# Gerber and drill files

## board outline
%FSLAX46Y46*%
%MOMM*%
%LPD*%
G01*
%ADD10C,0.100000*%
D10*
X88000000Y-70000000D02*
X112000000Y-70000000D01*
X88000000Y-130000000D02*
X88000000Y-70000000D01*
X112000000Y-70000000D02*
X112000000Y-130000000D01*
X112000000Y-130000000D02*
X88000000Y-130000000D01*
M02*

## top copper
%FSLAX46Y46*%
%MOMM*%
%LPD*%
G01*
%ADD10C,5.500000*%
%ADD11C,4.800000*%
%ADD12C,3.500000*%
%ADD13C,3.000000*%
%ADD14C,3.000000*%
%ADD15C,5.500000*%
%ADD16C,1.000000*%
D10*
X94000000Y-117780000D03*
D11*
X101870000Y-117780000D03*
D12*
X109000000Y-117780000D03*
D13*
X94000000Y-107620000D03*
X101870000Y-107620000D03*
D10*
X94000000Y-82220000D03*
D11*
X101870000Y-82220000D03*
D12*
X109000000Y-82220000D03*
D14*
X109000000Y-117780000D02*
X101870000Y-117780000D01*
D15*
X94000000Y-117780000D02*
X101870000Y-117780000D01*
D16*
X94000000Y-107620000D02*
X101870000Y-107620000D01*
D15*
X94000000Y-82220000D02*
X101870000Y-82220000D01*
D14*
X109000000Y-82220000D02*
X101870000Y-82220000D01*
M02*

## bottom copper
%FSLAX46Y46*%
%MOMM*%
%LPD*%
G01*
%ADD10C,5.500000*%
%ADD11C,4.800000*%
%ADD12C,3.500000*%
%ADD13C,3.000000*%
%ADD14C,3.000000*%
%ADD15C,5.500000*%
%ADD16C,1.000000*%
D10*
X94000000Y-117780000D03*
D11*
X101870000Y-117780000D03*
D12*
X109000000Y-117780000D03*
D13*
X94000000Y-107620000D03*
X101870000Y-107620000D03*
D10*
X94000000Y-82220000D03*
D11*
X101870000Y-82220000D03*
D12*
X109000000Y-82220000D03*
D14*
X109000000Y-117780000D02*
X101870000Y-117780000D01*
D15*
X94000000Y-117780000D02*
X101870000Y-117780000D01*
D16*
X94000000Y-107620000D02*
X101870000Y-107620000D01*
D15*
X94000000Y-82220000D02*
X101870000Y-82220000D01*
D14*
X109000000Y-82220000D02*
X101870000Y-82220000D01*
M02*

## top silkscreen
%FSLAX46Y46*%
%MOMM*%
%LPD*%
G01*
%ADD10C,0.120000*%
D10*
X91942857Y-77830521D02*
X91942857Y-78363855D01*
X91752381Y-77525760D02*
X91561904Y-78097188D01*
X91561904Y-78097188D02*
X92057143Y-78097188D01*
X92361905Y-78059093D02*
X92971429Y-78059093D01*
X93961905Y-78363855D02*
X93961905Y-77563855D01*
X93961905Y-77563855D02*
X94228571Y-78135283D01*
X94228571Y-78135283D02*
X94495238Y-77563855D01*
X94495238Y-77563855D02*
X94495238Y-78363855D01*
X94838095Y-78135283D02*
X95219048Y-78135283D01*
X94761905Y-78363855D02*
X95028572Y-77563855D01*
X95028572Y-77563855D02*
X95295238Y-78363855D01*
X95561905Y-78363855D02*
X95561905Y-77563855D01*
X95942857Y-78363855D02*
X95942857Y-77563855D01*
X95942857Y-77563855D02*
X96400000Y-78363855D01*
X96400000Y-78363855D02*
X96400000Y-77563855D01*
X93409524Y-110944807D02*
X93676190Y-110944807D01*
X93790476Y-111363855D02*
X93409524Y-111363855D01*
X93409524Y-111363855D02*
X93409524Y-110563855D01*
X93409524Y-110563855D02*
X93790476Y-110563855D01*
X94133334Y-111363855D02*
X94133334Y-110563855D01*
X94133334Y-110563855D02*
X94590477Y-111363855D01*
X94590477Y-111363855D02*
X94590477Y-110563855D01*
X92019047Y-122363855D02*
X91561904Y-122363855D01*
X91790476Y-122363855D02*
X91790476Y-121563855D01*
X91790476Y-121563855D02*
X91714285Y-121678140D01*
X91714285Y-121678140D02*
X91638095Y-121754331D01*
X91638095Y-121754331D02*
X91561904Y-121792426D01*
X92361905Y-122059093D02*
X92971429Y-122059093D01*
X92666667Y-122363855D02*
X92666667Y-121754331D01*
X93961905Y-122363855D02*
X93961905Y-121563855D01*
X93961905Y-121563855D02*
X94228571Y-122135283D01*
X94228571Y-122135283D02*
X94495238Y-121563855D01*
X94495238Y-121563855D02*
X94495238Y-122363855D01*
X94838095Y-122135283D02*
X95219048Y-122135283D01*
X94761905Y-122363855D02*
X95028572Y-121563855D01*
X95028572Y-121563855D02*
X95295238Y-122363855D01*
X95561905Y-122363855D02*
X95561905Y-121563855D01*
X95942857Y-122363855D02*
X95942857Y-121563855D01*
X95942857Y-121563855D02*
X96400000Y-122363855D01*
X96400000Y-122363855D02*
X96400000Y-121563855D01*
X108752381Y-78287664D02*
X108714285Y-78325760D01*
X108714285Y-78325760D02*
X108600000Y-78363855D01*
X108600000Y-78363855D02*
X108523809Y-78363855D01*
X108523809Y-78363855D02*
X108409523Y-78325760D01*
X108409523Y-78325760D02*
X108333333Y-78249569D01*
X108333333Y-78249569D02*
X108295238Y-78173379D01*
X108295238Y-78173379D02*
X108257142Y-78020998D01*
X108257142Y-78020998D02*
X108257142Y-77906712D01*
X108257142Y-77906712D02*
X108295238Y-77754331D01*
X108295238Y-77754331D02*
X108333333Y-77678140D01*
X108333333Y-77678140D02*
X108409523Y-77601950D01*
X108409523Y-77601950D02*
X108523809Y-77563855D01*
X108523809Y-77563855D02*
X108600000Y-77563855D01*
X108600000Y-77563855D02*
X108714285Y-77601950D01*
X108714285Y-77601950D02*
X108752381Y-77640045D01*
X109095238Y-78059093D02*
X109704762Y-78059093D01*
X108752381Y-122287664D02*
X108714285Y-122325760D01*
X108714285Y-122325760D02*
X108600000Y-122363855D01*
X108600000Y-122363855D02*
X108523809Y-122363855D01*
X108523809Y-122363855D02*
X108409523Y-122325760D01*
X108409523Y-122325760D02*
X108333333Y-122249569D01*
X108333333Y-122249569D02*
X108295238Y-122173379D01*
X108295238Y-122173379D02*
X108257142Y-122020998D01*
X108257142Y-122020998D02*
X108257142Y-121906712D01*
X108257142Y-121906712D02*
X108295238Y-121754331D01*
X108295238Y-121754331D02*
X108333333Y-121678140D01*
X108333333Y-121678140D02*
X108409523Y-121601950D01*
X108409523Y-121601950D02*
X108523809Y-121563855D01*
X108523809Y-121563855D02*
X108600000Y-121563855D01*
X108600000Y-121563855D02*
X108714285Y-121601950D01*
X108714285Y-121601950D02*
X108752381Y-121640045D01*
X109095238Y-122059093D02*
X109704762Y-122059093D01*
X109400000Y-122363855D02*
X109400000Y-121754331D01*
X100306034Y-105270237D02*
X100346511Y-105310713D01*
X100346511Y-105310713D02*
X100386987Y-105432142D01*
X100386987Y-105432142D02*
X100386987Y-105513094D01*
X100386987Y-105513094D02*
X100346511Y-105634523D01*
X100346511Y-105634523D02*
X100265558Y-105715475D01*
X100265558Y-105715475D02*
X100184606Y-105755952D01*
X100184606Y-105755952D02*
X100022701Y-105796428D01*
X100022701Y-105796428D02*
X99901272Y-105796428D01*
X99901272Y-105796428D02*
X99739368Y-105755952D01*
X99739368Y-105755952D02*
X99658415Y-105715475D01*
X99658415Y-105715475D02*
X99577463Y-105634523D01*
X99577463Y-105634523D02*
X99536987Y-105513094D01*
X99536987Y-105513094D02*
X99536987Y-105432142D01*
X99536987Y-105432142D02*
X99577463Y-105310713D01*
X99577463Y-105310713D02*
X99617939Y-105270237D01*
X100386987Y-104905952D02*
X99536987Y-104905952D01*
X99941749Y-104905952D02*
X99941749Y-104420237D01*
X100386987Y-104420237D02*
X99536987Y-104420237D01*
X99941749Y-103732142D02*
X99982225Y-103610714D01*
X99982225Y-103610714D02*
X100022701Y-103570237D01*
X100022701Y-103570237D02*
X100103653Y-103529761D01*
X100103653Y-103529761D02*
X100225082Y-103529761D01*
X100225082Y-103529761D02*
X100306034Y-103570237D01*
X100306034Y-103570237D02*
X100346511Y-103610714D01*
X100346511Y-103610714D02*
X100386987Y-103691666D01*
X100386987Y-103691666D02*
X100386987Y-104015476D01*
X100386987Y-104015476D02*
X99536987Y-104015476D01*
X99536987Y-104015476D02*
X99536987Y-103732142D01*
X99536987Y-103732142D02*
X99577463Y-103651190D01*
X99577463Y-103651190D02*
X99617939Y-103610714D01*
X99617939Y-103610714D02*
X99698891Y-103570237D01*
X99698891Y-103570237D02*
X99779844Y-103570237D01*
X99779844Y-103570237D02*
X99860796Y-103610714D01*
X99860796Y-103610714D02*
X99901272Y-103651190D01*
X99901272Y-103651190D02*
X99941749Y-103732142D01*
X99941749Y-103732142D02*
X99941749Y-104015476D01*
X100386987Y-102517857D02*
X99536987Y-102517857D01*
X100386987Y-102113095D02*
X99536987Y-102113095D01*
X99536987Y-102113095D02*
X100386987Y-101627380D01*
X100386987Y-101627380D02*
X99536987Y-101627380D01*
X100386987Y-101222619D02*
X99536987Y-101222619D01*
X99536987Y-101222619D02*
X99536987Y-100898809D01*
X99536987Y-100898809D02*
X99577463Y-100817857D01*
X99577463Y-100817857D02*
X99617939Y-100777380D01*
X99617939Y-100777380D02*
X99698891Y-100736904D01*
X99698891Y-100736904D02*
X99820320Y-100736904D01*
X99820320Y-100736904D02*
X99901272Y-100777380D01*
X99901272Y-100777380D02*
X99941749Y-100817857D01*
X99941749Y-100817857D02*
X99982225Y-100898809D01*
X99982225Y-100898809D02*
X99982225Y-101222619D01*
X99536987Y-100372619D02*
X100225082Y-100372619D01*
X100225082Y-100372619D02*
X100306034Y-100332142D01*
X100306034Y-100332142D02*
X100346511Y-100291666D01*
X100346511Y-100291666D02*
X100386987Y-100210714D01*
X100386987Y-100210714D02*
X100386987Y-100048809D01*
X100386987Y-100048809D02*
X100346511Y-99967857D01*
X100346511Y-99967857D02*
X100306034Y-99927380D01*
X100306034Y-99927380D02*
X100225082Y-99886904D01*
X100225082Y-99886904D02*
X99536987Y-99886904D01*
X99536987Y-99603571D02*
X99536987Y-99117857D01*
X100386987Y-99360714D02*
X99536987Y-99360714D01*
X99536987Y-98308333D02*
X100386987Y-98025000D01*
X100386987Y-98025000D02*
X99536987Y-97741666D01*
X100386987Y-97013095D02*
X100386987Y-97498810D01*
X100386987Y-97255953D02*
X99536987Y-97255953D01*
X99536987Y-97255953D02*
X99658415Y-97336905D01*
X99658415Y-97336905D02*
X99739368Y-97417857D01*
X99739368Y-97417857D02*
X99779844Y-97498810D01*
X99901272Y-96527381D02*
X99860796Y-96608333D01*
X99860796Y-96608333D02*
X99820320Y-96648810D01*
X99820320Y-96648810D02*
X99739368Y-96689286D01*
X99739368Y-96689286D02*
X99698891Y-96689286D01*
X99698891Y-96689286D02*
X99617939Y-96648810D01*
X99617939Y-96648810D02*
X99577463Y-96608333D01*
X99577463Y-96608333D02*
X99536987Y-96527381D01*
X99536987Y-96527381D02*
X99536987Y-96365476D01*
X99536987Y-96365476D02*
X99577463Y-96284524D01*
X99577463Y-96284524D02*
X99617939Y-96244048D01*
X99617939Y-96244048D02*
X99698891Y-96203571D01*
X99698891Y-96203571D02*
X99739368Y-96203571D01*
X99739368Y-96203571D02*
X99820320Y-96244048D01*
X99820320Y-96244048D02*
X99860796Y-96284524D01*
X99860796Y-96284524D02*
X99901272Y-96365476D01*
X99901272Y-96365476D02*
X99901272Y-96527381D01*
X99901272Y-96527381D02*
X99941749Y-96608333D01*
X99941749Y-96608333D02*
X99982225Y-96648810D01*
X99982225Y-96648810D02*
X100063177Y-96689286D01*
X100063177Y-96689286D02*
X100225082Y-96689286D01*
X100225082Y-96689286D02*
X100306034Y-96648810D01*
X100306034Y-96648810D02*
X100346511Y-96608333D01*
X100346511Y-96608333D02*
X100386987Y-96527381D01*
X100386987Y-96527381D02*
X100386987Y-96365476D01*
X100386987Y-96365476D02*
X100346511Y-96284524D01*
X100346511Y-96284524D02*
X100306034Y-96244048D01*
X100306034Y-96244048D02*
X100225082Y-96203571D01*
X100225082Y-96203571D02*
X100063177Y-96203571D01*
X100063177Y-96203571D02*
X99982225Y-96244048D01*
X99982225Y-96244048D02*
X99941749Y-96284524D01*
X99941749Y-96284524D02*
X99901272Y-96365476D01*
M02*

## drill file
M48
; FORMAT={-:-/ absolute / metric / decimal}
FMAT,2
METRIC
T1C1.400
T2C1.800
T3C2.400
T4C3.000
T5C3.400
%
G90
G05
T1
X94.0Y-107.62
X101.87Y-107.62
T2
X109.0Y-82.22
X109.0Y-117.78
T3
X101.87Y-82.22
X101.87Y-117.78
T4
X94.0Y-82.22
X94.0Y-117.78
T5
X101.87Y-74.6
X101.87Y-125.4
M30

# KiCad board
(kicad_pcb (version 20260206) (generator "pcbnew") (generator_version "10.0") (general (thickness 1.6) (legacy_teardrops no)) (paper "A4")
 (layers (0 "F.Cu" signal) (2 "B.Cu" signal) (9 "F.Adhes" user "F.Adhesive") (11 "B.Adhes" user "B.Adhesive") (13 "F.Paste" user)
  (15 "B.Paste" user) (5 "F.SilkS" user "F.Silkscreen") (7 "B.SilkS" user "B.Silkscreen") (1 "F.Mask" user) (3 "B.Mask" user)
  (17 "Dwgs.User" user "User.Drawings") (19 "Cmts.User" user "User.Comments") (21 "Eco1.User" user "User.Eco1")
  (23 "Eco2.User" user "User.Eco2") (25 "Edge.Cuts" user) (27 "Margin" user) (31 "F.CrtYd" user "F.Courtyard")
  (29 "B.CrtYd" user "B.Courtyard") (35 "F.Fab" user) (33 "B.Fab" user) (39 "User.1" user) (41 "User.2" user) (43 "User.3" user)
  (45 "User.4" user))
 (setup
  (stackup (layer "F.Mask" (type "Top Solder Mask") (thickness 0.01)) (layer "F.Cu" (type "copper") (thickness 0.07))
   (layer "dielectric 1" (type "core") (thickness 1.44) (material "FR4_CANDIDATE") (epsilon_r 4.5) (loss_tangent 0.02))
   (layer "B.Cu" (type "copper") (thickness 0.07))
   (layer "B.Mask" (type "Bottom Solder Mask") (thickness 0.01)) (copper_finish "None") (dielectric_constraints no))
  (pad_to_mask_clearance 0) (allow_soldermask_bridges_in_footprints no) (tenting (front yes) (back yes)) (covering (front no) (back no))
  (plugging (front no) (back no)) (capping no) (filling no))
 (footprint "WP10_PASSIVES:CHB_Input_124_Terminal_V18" (layer "F.Cu") (at 100 100)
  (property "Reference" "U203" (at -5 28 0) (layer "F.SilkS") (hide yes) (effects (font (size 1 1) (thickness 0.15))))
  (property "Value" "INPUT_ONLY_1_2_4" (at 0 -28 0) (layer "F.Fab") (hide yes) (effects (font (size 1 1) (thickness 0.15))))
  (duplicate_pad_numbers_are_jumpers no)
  (pad "" np_thru_hole circle (at 1.87 -25.4) (size 3.4 3.4) (drill 3.4) (layers "*.Cu" "*.Mask"))
  (pad "" np_thru_hole circle (at 1.87 25.4) (size 3.4 3.4) (drill 3.4) (layers "*.Cu" "*.Mask"))
  (pad "1" thru_hole circle (at -6 17.78) (size 5.5 5.5) (drill 3) (layers "*.Cu" "*.Mask") (remove_unused_layers no)
   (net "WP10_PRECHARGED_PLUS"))
  (pad "1" thru_hole circle (at 1.87 17.78) (size 4.8 4.8) (drill 2.4) (layers "*.Cu" "*.Mask") (remove_unused_layers no)
   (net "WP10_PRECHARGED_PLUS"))
  (pad "1" thru_hole circle (at 9 17.78) (size 3.5 3.5) (drill 1.8) (layers "*.Cu" "*.Mask") (remove_unused_layers no)
   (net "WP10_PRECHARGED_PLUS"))
  (pad "2" thru_hole circle (at -6 7.62) (size 3 3) (drill 1.4) (layers "*.Cu" "*.Mask") (remove_unused_layers no) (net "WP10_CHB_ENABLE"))
  (pad "2" thru_hole circle (at 1.87 7.62) (size 3 3) (drill 1.4) (layers "*.Cu" "*.Mask") (remove_unused_layers no) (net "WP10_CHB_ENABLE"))
  (pad "4" thru_hole circle (at -6 -17.78) (size 5.5 5.5) (drill 3) (layers "*.Cu" "*.Mask") (remove_unused_layers no)
   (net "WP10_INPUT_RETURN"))
  (pad "4" thru_hole circle (at 1.87 -17.78) (size 4.8 4.8) (drill 2.4) (layers "*.Cu" "*.Mask") (remove_unused_layers no)
   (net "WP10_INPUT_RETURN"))
  (pad "4" thru_hole circle (at 9 -17.78) (size 3.5 3.5) (drill 1.8) (layers "*.Cu" "*.Mask") (remove_unused_layers no)
   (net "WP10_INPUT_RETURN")))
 (gr_line (start 88 70) (end 112 70) (stroke (width 0.1) (type default)) (layer "Edge.Cuts"))
 (gr_line (start 88 130) (end 88 70) (stroke (width 0.1) (type default)) (layer "Edge.Cuts"))
 (gr_line (start 112 70) (end 112 130) (stroke (width 0.1) (type default)) (layer "Edge.Cuts"))
 (gr_line (start 112 130) (end 88 130) (stroke (width 0.1) (type default)) (layer "Edge.Cuts"))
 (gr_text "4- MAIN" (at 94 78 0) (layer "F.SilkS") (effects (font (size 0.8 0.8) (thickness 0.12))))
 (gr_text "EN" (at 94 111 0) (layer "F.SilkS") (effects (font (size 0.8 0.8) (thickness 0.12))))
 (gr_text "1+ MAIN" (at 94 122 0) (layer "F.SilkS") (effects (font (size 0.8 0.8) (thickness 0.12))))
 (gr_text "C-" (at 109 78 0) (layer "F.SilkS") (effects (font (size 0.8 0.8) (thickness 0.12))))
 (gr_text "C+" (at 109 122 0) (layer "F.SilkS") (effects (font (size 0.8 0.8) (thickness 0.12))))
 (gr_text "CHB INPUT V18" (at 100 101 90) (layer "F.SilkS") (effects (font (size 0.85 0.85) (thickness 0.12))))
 (segment (start 109 117.78) (end 101.87 117.78) (width 3) (layer "F.Cu") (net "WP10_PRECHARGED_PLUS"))
 (segment (start 94 117.78) (end 101.87 117.78) (width 5.5) (layer "F.Cu") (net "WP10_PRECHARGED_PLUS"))
 (segment (start 109 117.78) (end 101.87 117.78) (width 3) (layer "B.Cu") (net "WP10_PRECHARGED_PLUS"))
 (segment (start 94 117.78) (end 101.87 117.78) (width 5.5) (layer "B.Cu") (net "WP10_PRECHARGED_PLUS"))
 (segment (start 94 107.62) (end 101.87 107.62) (width 1) (layer "F.Cu") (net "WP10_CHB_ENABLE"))
 (segment (start 94 107.62) (end 101.87 107.62) (width 1) (layer "B.Cu") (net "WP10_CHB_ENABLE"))
 (segment (start 94 82.22) (end 101.87 82.22) (width 5.5) (layer "F.Cu") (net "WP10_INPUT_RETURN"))
 (segment (start 109 82.22) (end 101.87 82.22) (width 3) (layer "F.Cu") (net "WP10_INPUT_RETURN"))
 (segment (start 94 82.22) (end 101.87 82.22) (width 5.5) (layer "B.Cu") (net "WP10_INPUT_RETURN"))
 (segment (start 109 82.22) (end 101.87 82.22) (width 3) (layer "B.Cu") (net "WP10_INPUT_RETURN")))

